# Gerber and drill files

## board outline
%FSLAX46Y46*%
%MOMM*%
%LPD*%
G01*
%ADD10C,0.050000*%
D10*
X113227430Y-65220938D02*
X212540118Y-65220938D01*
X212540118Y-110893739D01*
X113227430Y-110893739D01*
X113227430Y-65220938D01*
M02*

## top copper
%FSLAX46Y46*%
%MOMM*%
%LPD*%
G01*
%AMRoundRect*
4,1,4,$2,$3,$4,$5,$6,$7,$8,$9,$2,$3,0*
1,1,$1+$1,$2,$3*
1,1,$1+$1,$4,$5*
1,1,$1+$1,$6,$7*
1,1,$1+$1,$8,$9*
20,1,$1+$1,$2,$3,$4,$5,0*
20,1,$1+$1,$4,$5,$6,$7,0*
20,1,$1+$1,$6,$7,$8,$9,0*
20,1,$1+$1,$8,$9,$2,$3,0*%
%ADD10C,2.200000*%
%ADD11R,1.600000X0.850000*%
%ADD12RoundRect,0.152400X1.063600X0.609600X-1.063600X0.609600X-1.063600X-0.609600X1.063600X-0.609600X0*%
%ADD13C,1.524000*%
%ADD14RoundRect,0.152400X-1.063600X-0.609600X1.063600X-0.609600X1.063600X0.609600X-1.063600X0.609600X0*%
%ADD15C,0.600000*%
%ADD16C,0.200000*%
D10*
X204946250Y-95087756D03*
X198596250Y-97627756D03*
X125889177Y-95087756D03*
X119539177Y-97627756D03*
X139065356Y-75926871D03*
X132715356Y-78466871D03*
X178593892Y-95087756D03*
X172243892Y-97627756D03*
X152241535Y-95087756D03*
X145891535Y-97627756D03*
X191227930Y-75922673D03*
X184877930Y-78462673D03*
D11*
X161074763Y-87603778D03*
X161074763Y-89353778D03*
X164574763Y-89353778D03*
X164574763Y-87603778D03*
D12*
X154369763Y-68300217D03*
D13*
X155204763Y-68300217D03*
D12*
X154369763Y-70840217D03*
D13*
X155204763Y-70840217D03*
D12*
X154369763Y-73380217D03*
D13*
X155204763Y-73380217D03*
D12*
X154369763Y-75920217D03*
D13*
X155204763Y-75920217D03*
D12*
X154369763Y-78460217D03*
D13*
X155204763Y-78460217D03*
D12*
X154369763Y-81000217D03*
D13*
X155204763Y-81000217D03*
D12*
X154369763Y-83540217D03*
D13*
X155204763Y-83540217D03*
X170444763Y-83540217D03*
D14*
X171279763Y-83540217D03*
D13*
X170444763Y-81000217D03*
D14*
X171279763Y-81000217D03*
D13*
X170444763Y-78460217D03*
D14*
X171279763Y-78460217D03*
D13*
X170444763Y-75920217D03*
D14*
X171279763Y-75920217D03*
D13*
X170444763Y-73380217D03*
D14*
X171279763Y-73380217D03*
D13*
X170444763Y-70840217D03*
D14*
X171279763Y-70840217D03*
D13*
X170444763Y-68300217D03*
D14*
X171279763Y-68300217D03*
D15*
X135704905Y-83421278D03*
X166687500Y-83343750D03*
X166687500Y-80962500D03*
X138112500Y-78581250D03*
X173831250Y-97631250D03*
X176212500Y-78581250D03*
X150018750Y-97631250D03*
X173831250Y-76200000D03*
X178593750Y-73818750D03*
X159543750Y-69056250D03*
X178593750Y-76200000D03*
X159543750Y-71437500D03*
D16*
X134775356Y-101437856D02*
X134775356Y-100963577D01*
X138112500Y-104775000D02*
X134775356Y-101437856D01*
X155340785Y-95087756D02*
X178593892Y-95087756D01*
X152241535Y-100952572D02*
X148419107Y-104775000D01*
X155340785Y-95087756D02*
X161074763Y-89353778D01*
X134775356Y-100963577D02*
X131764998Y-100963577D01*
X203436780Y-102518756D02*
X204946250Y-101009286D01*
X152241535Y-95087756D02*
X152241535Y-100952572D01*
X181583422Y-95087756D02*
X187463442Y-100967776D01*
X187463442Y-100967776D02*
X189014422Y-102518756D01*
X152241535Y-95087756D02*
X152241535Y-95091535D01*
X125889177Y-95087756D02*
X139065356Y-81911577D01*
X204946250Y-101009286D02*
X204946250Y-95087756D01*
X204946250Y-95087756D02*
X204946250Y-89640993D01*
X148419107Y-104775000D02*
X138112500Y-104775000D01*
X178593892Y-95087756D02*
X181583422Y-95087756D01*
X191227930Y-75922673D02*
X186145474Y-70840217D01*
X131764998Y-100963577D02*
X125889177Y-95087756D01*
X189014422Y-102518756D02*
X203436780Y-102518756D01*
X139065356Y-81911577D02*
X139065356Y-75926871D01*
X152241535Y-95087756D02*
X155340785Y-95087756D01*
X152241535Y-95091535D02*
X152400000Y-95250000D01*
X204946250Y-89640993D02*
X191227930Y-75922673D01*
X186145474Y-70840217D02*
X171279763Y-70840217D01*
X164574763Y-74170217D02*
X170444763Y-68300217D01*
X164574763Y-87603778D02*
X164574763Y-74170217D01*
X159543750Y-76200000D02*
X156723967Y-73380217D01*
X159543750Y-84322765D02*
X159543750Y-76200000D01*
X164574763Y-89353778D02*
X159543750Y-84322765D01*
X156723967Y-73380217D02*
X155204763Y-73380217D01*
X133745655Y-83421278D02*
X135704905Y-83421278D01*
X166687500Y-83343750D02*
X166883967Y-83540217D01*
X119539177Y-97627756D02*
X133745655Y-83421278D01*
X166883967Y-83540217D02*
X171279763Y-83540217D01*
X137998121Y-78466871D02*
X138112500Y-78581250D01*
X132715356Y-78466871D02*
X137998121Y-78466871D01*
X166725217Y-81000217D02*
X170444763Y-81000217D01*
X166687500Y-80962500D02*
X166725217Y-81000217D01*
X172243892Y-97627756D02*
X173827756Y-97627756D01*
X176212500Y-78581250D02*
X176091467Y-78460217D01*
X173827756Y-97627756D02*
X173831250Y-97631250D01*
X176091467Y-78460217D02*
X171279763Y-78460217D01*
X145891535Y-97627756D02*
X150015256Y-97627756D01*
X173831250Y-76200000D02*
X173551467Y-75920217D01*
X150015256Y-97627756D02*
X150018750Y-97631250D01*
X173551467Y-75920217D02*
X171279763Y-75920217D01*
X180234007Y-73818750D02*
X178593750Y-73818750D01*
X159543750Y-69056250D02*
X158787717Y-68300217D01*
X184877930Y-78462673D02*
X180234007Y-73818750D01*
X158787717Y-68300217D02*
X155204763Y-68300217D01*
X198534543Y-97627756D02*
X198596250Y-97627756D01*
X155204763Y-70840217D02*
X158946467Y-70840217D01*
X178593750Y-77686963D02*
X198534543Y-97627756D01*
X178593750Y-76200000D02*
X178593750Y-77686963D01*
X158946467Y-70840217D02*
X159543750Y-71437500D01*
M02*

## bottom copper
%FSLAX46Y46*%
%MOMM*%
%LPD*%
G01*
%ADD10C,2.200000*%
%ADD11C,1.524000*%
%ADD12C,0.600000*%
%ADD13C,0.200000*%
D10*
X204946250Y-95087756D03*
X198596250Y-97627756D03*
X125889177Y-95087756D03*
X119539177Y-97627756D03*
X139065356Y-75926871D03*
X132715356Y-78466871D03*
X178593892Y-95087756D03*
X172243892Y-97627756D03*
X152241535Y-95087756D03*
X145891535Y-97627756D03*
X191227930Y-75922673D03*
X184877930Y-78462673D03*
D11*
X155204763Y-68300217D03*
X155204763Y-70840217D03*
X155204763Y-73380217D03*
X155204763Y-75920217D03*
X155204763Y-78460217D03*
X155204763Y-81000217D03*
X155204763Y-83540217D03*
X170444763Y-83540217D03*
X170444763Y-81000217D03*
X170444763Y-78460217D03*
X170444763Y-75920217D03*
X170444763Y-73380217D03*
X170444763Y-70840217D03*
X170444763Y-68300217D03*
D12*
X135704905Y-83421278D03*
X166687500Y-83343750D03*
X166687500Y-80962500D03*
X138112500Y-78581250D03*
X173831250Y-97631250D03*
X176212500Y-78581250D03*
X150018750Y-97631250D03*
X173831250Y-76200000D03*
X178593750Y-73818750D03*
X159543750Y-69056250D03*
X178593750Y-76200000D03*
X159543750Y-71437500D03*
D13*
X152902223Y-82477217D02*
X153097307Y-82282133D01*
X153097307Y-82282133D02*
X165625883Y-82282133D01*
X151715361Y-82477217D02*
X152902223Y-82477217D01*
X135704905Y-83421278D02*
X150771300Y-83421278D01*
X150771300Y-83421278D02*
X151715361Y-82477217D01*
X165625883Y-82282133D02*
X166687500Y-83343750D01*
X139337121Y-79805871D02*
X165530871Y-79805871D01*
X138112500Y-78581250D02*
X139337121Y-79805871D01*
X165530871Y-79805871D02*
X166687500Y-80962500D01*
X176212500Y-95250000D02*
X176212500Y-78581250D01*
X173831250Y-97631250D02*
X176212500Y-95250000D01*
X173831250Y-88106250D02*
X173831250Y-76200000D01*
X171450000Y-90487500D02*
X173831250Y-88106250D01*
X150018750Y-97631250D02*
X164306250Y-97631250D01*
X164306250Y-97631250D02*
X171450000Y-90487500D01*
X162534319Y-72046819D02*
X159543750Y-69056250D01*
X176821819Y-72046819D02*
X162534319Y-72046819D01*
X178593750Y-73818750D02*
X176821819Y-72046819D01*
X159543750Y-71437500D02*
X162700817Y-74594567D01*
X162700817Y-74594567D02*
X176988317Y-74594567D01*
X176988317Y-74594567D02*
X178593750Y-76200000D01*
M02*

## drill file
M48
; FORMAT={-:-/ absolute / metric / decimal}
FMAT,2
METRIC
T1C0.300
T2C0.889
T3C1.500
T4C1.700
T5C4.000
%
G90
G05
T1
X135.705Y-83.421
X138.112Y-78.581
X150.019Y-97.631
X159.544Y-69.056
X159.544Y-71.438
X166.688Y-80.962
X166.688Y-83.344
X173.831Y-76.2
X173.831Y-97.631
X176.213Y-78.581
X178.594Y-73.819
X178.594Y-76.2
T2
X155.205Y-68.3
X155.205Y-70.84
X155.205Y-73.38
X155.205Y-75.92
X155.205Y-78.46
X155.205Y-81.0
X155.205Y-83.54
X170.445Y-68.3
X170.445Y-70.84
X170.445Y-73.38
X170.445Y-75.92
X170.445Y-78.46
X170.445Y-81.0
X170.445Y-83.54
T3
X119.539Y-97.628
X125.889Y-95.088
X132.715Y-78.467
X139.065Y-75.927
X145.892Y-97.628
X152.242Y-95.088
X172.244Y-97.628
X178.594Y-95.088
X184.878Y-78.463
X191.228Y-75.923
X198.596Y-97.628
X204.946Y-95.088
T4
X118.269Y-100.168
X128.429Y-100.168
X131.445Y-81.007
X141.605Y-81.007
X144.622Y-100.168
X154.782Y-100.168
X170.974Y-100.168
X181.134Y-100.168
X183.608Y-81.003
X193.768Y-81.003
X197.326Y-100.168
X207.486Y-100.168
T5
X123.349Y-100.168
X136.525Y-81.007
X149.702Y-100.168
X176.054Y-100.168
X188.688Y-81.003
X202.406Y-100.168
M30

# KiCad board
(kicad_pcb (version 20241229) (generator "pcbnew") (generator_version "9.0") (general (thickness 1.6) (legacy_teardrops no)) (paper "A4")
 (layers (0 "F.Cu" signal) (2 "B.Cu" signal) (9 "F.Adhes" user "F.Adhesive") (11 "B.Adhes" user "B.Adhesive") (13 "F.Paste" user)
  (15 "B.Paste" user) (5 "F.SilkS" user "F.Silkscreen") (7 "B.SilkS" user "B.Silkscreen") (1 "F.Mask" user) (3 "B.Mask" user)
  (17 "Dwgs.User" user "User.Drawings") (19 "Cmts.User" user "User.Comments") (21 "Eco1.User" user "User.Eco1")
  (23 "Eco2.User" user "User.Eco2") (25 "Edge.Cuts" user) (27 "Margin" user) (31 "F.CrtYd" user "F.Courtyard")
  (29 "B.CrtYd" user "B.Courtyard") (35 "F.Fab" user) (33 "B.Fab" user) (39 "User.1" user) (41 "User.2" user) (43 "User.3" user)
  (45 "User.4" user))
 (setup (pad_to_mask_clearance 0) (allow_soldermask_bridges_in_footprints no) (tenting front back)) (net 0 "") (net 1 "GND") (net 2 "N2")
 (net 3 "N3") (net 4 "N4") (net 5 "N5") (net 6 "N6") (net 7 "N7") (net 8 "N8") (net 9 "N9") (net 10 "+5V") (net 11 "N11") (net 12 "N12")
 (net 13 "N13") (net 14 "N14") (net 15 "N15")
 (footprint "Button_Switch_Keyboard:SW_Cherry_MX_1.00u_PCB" (layer "F.Cu") (at 204.94625 95.087756)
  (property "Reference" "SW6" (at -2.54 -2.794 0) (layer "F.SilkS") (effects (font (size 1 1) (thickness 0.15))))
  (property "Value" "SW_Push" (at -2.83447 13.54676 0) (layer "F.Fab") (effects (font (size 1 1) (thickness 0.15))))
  (pad "" np_thru_hole circle (at -7.62 5.08) (size 1.7 1.7) (drill 1.7) (layers "*.Cu" "*.Mask"))
  (pad "" np_thru_hole circle (at -2.54 5.08) (size 4 4) (drill 4) (layers "*.Cu" "*.Mask"))
  (pad "" np_thru_hole circle (at 2.54 5.08) (size 1.7 1.7) (drill 1.7) (layers "*.Cu" "*.Mask"))
  (pad "1" thru_hole circle (at 0 0) (size 2.2 2.2) (drill 1.5) (layers "*.Cu" "*.Mask") (remove_unused_layers no) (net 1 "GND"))
  (pad "2" thru_hole circle (at -6.35 2.54) (size 2.2 2.2) (drill 1.5) (layers "*.Cu" "*.Mask") (remove_unused_layers no) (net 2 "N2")))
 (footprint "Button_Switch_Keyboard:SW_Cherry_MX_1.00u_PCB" (layer "F.Cu") (at 125.889177 95.087756)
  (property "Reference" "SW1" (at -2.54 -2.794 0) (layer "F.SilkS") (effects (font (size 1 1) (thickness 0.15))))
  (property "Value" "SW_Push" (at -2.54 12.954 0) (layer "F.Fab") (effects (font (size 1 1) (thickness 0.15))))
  (pad "" np_thru_hole circle (at -7.62 5.08) (size 1.7 1.7) (drill 1.7) (layers "*.Cu" "*.Mask"))
  (pad "" np_thru_hole circle (at -2.54 5.08) (size 4 4) (drill 4) (layers "*.Cu" "*.Mask"))
  (pad "" np_thru_hole circle (at 2.54 5.08) (size 1.7 1.7) (drill 1.7) (layers "*.Cu" "*.Mask"))
  (pad "1" thru_hole circle (at 0 0) (size 2.2 2.2) (drill 1.5) (layers "*.Cu" "*.Mask") (remove_unused_layers no) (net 1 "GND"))
  (pad "2" thru_hole circle (at -6.35 2.54) (size 2.2 2.2) (drill 1.5) (layers "*.Cu" "*.Mask") (remove_unused_layers no) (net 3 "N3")))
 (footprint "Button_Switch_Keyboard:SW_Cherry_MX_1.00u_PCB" (layer "F.Cu") (at 139.065356 75.926871)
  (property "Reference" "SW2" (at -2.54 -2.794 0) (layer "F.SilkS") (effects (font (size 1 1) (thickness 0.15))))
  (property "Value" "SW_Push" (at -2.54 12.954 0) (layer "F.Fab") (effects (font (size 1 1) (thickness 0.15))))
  (pad "" np_thru_hole circle (at -7.62 5.08) (size 1.7 1.7) (drill 1.7) (layers "*.Cu" "*.Mask"))
  (pad "" np_thru_hole circle (at -2.54 5.08) (size 4 4) (drill 4) (layers "*.Cu" "*.Mask"))
  (pad "" np_thru_hole circle (at 2.54 5.08) (size 1.7 1.7) (drill 1.7) (layers "*.Cu" "*.Mask"))
  (pad "1" thru_hole circle (at 0 0) (size 2.2 2.2) (drill 1.5) (layers "*.Cu" "*.Mask") (remove_unused_layers no) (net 1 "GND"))
  (pad "2" thru_hole circle (at -6.35 2.54) (size 2.2 2.2) (drill 1.5) (layers "*.Cu" "*.Mask") (remove_unused_layers no) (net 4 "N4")))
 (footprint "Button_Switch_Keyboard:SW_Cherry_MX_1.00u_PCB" (layer "F.Cu") (at 178.593892 95.087756)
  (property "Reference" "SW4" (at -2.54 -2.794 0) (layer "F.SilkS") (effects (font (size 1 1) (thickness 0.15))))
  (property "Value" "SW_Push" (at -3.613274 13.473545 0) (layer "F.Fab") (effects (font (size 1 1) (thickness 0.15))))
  (pad "" np_thru_hole circle (at -7.62 5.08) (size 1.7 1.7) (drill 1.7) (layers "*.Cu" "*.Mask"))
  (pad "" np_thru_hole circle (at -2.54 5.08) (size 4 4) (drill 4) (layers "*.Cu" "*.Mask"))
  (pad "" np_thru_hole circle (at 2.54 5.08) (size 1.7 1.7) (drill 1.7) (layers "*.Cu" "*.Mask"))
  (pad "1" thru_hole circle (at 0 0) (size 2.2 2.2) (drill 1.5) (layers "*.Cu" "*.Mask") (remove_unused_layers no) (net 1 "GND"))
  (pad "2" thru_hole circle (at -6.35 2.54) (size 2.2 2.2) (drill 1.5) (layers "*.Cu" "*.Mask") (remove_unused_layers no) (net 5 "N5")))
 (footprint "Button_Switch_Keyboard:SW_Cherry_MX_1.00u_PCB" (layer "F.Cu") (at 152.241535 95.087756)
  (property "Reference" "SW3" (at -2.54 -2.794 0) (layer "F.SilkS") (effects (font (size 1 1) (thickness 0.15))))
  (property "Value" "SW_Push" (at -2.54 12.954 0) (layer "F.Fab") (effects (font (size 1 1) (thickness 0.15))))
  (pad "" np_thru_hole circle (at -7.62 5.08) (size 1.7 1.7) (drill 1.7) (layers "*.Cu" "*.Mask"))
  (pad "" np_thru_hole circle (at -2.54 5.08) (size 4 4) (drill 4) (layers "*.Cu" "*.Mask"))
  (pad "" np_thru_hole circle (at 2.54 5.08) (size 1.7 1.7) (drill 1.7) (layers "*.Cu" "*.Mask"))
  (pad "1" thru_hole circle (at 0 0) (size 2.2 2.2) (drill 1.5) (layers "*.Cu" "*.Mask") (remove_unused_layers no) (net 1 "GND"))
  (pad "2" thru_hole circle (at -6.35 2.54) (size 2.2 2.2) (drill 1.5) (layers "*.Cu" "*.Mask") (remove_unused_layers no) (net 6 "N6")))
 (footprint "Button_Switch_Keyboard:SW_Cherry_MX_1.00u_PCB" (layer "F.Cu") (at 191.22793 75.922673)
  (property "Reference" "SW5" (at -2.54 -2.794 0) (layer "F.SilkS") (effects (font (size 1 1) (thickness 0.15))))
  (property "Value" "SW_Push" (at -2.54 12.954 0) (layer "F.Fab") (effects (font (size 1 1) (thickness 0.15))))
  (pad "" np_thru_hole circle (at -7.62 5.08) (size 1.7 1.7) (drill 1.7) (layers "*.Cu" "*.Mask"))
  (pad "" np_thru_hole circle (at -2.54 5.08) (size 4 4) (drill 4) (layers "*.Cu" "*.Mask"))
  (pad "" np_thru_hole circle (at 2.54 5.08) (size 1.7 1.7) (drill 1.7) (layers "*.Cu" "*.Mask"))
  (pad "1" thru_hole circle (at 0 0) (size 2.2 2.2) (drill 1.5) (layers "*.Cu" "*.Mask") (remove_unused_layers no) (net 1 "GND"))
  (pad "2" thru_hole circle (at -6.35 2.54) (size 2.2 2.2) (drill 1.5) (layers "*.Cu" "*.Mask") (remove_unused_layers no) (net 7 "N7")))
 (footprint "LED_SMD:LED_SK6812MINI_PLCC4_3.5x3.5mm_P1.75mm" (layer "F.Cu") (at 162.824763 88.478778)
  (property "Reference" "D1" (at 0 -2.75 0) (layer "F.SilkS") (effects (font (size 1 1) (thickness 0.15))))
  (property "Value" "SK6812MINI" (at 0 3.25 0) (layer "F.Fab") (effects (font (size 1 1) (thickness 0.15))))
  (pad "1" smd rect (at -1.75 -0.875) (size 1.6 0.85) (layers "F.Cu" "F.Mask" "F.Paste") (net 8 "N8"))
  (pad "2" smd rect (at -1.75 0.875) (size 1.6 0.85) (layers "F.Cu" "F.Mask" "F.Paste") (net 1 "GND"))
  (pad "3" smd rect (at 1.75 0.875) (size 1.6 0.85) (layers "F.Cu" "F.Mask" "F.Paste") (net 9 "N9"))
  (pad "4" smd rect (at 1.75 -0.875) (size 1.6 0.85) (layers "F.Cu" "F.Mask" "F.Paste") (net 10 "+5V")))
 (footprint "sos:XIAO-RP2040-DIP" (layer "F.Cu") (at 162.824763 75.920217)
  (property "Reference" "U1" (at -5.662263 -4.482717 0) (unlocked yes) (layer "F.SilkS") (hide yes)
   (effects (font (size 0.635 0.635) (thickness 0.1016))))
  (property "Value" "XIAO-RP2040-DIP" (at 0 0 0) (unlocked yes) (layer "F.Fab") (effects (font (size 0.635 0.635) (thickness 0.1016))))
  (pad "1" smd roundrect (at -8.455 -7.62 180) (size 2.432 1.524) (layers "F.Cu" "F.Mask") (roundrect_rratio 0.1) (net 7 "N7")
   (thermal_bridge_angle 45))
  (pad "1" thru_hole circle (at -7.62 -7.62 180) (size 1.524 1.524) (drill 0.889) (layers "*.Cu" "*.Mask") (remove_unused_layers no)
   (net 7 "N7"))
  (pad "2" smd roundrect (at -8.455 -5.08 180) (size 2.432 1.524) (layers "F.Cu" "F.Mask") (roundrect_rratio 0.1) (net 2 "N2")
   (thermal_bridge_angle 45))
  (pad "2" thru_hole circle (at -7.62 -5.08 180) (size 1.524 1.524) (drill 0.889) (layers "*.Cu" "*.Mask") (remove_unused_layers no)
   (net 2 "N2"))
  (pad "3" smd roundrect (at -8.455 -2.54 180) (size 2.432 1.524) (layers "F.Cu" "F.Mask") (roundrect_rratio 0.1) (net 9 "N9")
   (thermal_bridge_angle 45))
  (pad "3" thru_hole circle (at -7.62 -2.54 180) (size 1.524 1.524) (drill 0.889) (layers "*.Cu" "*.Mask") (remove_unused_layers no)
   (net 9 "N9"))
  (pad "4" smd roundrect (at -8.455 0 180) (size 2.432 1.524) (layers "F.Cu" "F.Mask") (roundrect_rratio 0.1) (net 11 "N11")
   (thermal_bridge_angle 45))
  (pad "4" thru_hole circle (at -7.62 0 180) (size 1.524 1.524) (drill 0.889) (layers "*.Cu" "*.Mask") (remove_unused_layers no)
   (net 11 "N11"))
  (pad "5" smd roundrect (at -8.455 2.54 180) (size 2.432 1.524) (layers "F.Cu" "F.Mask") (roundrect_rratio 0.1) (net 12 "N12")
   (thermal_bridge_angle 45))
  (pad "5" thru_hole circle (at -7.62 2.54 180) (size 1.524 1.524) (drill 0.889) (layers "*.Cu" "*.Mask") (remove_unused_layers no)
   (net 12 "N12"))
  (pad "6" smd roundrect (at -8.455 5.08 180) (size 2.432 1.524) (layers "F.Cu" "F.Mask") (roundrect_rratio 0.1) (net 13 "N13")
   (thermal_bridge_angle 45))
  (pad "6" thru_hole circle (at -7.62 5.08 180) (size 1.524 1.524) (drill 0.889) (layers "*.Cu" "*.Mask") (remove_unused_layers no)
   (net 13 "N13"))
  (pad "7" smd roundrect (at -8.455 7.62 180) (size 2.432 1.524) (layers "F.Cu" "F.Mask") (roundrect_rratio 0.1) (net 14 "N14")
   (thermal_bridge_angle 45))
  (pad "7" thru_hole circle (at -7.62 7.62 180) (size 1.524 1.524) (drill 0.889) (layers "*.Cu" "*.Mask") (remove_unused_layers no)
   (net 14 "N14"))
  (pad "8" thru_hole circle (at 7.62 7.62) (size 1.524 1.524) (drill 0.889) (layers "*.Cu" "*.Mask") (remove_unused_layers no) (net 3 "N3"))
  (pad "8" smd roundrect (at 8.455 7.62) (size 2.432 1.524) (layers "F.Cu" "F.Mask") (roundrect_rratio 0.1) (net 3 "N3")
   (thermal_bridge_angle 45))
  (pad "9" thru_hole circle (at 7.62 5.08) (size 1.524 1.524) (drill 0.889) (layers "*.Cu" "*.Mask") (remove_unused_layers no) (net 4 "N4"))
  (pad "9" smd roundrect (at 8.455 5.08) (size 2.432 1.524) (layers "F.Cu" "F.Mask") (roundrect_rratio 0.1) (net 4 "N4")
   (thermal_bridge_angle 45))
  (pad "10" thru_hole circle (at 7.62 2.54) (size 1.524 1.524) (drill 0.889) (layers "*.Cu" "*.Mask") (remove_unused_layers no) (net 5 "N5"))
  (pad "10" smd roundrect (at 8.455 2.54) (size 2.432 1.524) (layers "F.Cu" "F.Mask") (roundrect_rratio 0.1) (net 5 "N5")
   (thermal_bridge_angle 45))
  (pad "11" thru_hole circle (at 7.62 0) (size 1.524 1.524) (drill 0.889) (layers "*.Cu" "*.Mask") (remove_unused_layers no) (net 6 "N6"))
  (pad "11" smd roundrect (at 8.455 0) (size 2.432 1.524) (layers "F.Cu" "F.Mask") (roundrect_rratio 0.1) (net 6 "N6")
   (thermal_bridge_angle 45))
  (pad "12" thru_hole circle (at 7.62 -2.54) (size 1.524 1.524) (drill 0.889) (layers "*.Cu" "*.Mask") (remove_unused_layers no)
   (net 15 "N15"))
  (pad "12" smd roundrect (at 8.455 -2.54) (size 2.432 1.524) (layers "F.Cu" "F.Mask") (roundrect_rratio 0.1) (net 15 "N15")
   (thermal_bridge_angle 45))
  (pad "13" thru_hole circle (at 7.62 -5.08) (size 1.524 1.524) (drill 0.889) (layers "*.Cu" "*.Mask") (remove_unused_layers no)
   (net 1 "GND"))
  (pad "13" smd roundrect (at 8.455 -5.08) (size 2.432 1.524) (layers "F.Cu" "F.Mask") (roundrect_rratio 0.1) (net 1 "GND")
   (thermal_bridge_angle 45))
  (pad "14" thru_hole circle (at 7.62 -7.62) (size 1.524 1.524) (drill 0.889) (layers "*.Cu" "*.Mask") (remove_unused_layers no)
   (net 10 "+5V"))
  (pad "14" smd roundrect (at 8.455 -7.62) (size 2.432 1.524) (layers "F.Cu" "F.Mask") (roundrect_rratio 0.1) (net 10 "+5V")
   (thermal_bridge_angle 45)))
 (gr_rect (start 113.22743 65.220938) (end 212.540118 110.893739) (stroke (width 0.05) (type default)) (fill no) (layer "Edge.Cuts"))
 (segment (start 134.775356 101.437856) (end 134.775356 100.963577) (width 0.2) (layer "F.Cu") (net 1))
 (segment (start 138.1125 104.775) (end 134.775356 101.437856) (width 0.2) (layer "F.Cu") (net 1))
 (segment (start 155.340785 95.087756) (end 178.593892 95.087756) (width 0.2) (layer "F.Cu") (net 1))
 (segment (start 152.241535 100.952572) (end 148.419107 104.775) (width 0.2) (layer "F.Cu") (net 1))
 (segment (start 155.340785 95.087756) (end 161.074763 89.353778) (width 0.2) (layer "F.Cu") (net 1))
 (segment (start 134.775356 100.963577) (end 131.764998 100.963577) (width 0.2) (layer "F.Cu") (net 1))
 (segment (start 203.43678 102.518756) (end 204.94625 101.009286) (width 0.2) (layer "F.Cu") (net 1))
 (segment (start 152.241535 95.087756) (end 152.241535 100.952572) (width 0.2) (layer "F.Cu") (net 1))
 (segment (start 181.583422 95.087756) (end 187.463442 100.967776) (width 0.2) (layer "F.Cu") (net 1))
 (segment (start 187.463442 100.967776) (end 189.014422 102.518756) (width 0.2) (layer "F.Cu") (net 1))
 (segment (start 152.241535 95.087756) (end 152.241535 95.091535) (width 0.2) (layer "F.Cu") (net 1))
 (segment (start 125.889177 95.087756) (end 139.065356 81.911577) (width 0.2) (layer "F.Cu") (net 1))
 (segment (start 204.94625 101.009286) (end 204.94625 95.087756) (width 0.2) (layer "F.Cu") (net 1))
 (segment (start 204.94625 95.087756) (end 204.94625 89.640993) (width 0.2) (layer "F.Cu") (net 1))
 (segment (start 148.419107 104.775) (end 138.1125 104.775) (width 0.2) (layer "F.Cu") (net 1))
 (segment (start 178.593892 95.087756) (end 181.583422 95.087756) (width 0.2) (layer "F.Cu") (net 1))
 (segment (start 191.22793 75.922673) (end 186.145474 70.840217) (width 0.2) (layer "F.Cu") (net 1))
 (segment (start 131.764998 100.963577) (end 125.889177 95.087756) (width 0.2) (layer "F.Cu") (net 1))
 (segment (start 189.014422 102.518756) (end 203.43678 102.518756) (width 0.2) (layer "F.Cu") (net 1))
 (segment (start 139.065356 81.911577) (end 139.065356 75.926871) (width 0.2) (layer "F.Cu") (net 1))
 (segment (start 152.241535 95.087756) (end 155.340785 95.087756) (width 0.2) (layer "F.Cu") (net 1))
 (segment (start 152.241535 95.091535) (end 152.4 95.25) (width 0.2) (layer "F.Cu") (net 1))
 (segment (start 204.94625 89.640993) (end 191.22793 75.922673) (width 0.2) (layer "F.Cu") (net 1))
 (segment (start 186.145474 70.840217) (end 171.279763 70.840217) (width 0.2) (layer "F.Cu") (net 1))
 (segment (start 164.574763 74.170217) (end 170.444763 68.300217) (width 0.2) (layer "F.Cu") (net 10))
 (segment (start 164.574763 87.603778) (end 164.574763 74.170217) (width 0.2) (layer "F.Cu") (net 10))
 (segment (start 159.54375 76.2) (end 156.723967 73.380217) (width 0.2) (layer "F.Cu") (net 9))
 (segment (start 159.54375 84.322765) (end 159.54375 76.2) (width 0.2) (layer "F.Cu") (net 9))
 (segment (start 164.574763 89.353778) (end 159.54375 84.322765) (width 0.2) (layer "F.Cu") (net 9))
 (segment (start 156.723967 73.380217) (end 155.204763 73.380217) (width 0.2) (layer "F.Cu") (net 9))
 (segment (start 133.745655 83.421278) (end 135.704905 83.421278) (width 0.2) (layer "F.Cu") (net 3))
 (segment (start 166.6875 83.34375) (end 166.883967 83.540217) (width 0.2) (layer "F.Cu") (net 3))
 (segment (start 119.539177 97.627756) (end 133.745655 83.421278) (width 0.2) (layer "F.Cu") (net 3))
 (segment (start 166.883967 83.540217) (end 171.279763 83.540217) (width 0.2) (layer "F.Cu") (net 3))
 (via (at 135.704905 83.421278) (size 0.6) (drill 0.3) (layers "F.Cu" "B.Cu") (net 3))
 (via (at 166.6875 83.34375) (size 0.6) (drill 0.3) (layers "F.Cu" "B.Cu") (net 3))
 (segment (start 152.902223 82.477217) (end 153.097307 82.282133) (width 0.2) (layer "B.Cu") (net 3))
 (segment (start 153.097307 82.282133) (end 165.625883 82.282133) (width 0.2) (layer "B.Cu") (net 3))
 (segment (start 151.715361 82.477217) (end 152.902223 82.477217) (width 0.2) (layer "B.Cu") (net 3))
 (segment (start 135.704905 83.421278) (end 150.7713 83.421278) (width 0.2) (layer "B.Cu") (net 3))
 (segment (start 150.7713 83.421278) (end 151.715361 82.477217) (width 0.2) (layer "B.Cu") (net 3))
 (segment (start 165.625883 82.282133) (end 166.6875 83.34375) (width 0.2) (layer "B.Cu") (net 3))
 (segment (start 137.998121 78.466871) (end 138.1125 78.58125) (width 0.2) (layer "F.Cu") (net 4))
 (segment (start 132.715356 78.466871) (end 137.998121 78.466871) (width 0.2) (layer "F.Cu") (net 4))
 (segment (start 166.725217 81.000217) (end 170.444763 81.000217) (width 0.2) (layer "F.Cu") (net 4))
 (segment (start 166.6875 80.9625) (end 166.725217 81.000217) (width 0.2) (layer "F.Cu") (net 4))
 (via (at 166.6875 80.9625) (size 0.6) (drill 0.3) (layers "F.Cu" "B.Cu") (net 4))
 (via (at 138.1125 78.58125) (size 0.6) (drill 0.3) (layers "F.Cu" "B.Cu") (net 4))
 (segment (start 139.337121 79.805871) (end 165.530871 79.805871) (width 0.2) (layer "B.Cu") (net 4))
 (segment (start 138.1125 78.58125) (end 139.337121 79.805871) (width 0.2) (layer "B.Cu") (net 4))
 (segment (start 165.530871 79.805871) (end 166.6875 80.9625) (width 0.2) (layer "B.Cu") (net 4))
 (segment (start 172.243892 97.627756) (end 173.827756 97.627756) (width 0.2) (layer "F.Cu") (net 5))
 (segment (start 176.2125 78.58125) (end 176.091467 78.460217) (width 0.2) (layer "F.Cu") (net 5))
 (segment (start 173.827756 97.627756) (end 173.83125 97.63125) (width 0.2) (layer "F.Cu") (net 5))
 (segment (start 176.091467 78.460217) (end 171.279763 78.460217) (width 0.2) (layer "F.Cu") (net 5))
 (via (at 173.83125 97.63125) (size 0.6) (drill 0.3) (layers "F.Cu" "B.Cu") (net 5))
 (via (at 176.2125 78.58125) (size 0.6) (drill 0.3) (layers "F.Cu" "B.Cu") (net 5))
 (segment (start 176.2125 95.25) (end 176.2125 78.58125) (width 0.2) (layer "B.Cu") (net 5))
 (segment (start 173.83125 97.63125) (end 176.2125 95.25) (width 0.2) (layer "B.Cu") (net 5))
 (segment (start 145.891535 97.627756) (end 150.015256 97.627756) (width 0.2) (layer "F.Cu") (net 6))
 (segment (start 173.83125 76.2) (end 173.551467 75.920217) (width 0.2) (layer "F.Cu") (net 6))
 (segment (start 150.015256 97.627756) (end 150.01875 97.63125) (width 0.2) (layer "F.Cu") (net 6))
 (segment (start 173.551467 75.920217) (end 171.279763 75.920217) (width 0.2) (layer "F.Cu") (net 6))
 (via (at 150.01875 97.63125) (size 0.6) (drill 0.3) (layers "F.Cu" "B.Cu") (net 6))
 (via (at 173.83125 76.2) (size 0.6) (drill 0.3) (layers "F.Cu" "B.Cu") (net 6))
 (segment (start 173.83125 88.10625) (end 173.83125 76.2) (width 0.2) (layer "B.Cu") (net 6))
 (segment (start 171.45 90.4875) (end 173.83125 88.10625) (width 0.2) (layer "B.Cu") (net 6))
 (segment (start 150.01875 97.63125) (end 164.30625 97.63125) (width 0.2) (layer "B.Cu") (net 6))
 (segment (start 164.30625 97.63125) (end 171.45 90.4875) (width 0.2) (layer "B.Cu") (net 6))
 (segment (start 180.234007 73.81875) (end 178.59375 73.81875) (width 0.2) (layer "F.Cu") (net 7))
 (segment (start 159.54375 69.05625) (end 158.787717 68.300217) (width 0.2) (layer "F.Cu") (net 7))
 (segment (start 184.87793 78.462673) (end 180.234007 73.81875) (width 0.2) (layer "F.Cu") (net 7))
 (segment (start 158.787717 68.300217) (end 155.204763 68.300217) (width 0.2) (layer "F.Cu") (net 7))
 (via (at 178.59375 73.81875) (size 0.6) (drill 0.3) (layers "F.Cu" "B.Cu") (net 7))
 (via (at 159.54375 69.05625) (size 0.6) (drill 0.3) (layers "F.Cu" "B.Cu") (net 7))
 (segment (start 162.534319 72.046819) (end 159.54375 69.05625) (width 0.2) (layer "B.Cu") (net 7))
 (segment (start 176.821819 72.046819) (end 162.534319 72.046819) (width 0.2) (layer "B.Cu") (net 7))
 (segment (start 178.59375 73.81875) (end 176.821819 72.046819) (width 0.2) (layer "B.Cu") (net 7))
 (segment (start 198.534543 97.627756) (end 198.59625 97.627756) (width 0.2) (layer "F.Cu") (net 2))
 (segment (start 155.204763 70.840217) (end 158.946467 70.840217) (width 0.2) (layer "F.Cu") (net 2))
 (segment (start 178.59375 77.686963) (end 198.534543 97.627756) (width 0.2) (layer "F.Cu") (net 2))
 (segment (start 178.59375 76.2) (end 178.59375 77.686963) (width 0.2) (layer "F.Cu") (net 2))
 (segment (start 158.946467 70.840217) (end 159.54375 71.4375) (width 0.2) (layer "F.Cu") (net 2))
 (via (at 178.59375 76.2) (size 0.6) (drill 0.3) (layers "F.Cu" "B.Cu") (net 2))
 (via (at 159.54375 71.4375) (size 0.6) (drill 0.3) (layers "F.Cu" "B.Cu") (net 2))
 (segment (start 159.54375 71.4375) (end 162.700817 74.594567) (width 0.2) (layer "B.Cu") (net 2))
 (segment (start 162.700817 74.594567) (end 176.988317 74.594567) (width 0.2) (layer "B.Cu") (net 2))
 (segment (start 176.988317 74.594567) (end 178.59375 76.2) (width 0.2) (layer "B.Cu") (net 2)))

